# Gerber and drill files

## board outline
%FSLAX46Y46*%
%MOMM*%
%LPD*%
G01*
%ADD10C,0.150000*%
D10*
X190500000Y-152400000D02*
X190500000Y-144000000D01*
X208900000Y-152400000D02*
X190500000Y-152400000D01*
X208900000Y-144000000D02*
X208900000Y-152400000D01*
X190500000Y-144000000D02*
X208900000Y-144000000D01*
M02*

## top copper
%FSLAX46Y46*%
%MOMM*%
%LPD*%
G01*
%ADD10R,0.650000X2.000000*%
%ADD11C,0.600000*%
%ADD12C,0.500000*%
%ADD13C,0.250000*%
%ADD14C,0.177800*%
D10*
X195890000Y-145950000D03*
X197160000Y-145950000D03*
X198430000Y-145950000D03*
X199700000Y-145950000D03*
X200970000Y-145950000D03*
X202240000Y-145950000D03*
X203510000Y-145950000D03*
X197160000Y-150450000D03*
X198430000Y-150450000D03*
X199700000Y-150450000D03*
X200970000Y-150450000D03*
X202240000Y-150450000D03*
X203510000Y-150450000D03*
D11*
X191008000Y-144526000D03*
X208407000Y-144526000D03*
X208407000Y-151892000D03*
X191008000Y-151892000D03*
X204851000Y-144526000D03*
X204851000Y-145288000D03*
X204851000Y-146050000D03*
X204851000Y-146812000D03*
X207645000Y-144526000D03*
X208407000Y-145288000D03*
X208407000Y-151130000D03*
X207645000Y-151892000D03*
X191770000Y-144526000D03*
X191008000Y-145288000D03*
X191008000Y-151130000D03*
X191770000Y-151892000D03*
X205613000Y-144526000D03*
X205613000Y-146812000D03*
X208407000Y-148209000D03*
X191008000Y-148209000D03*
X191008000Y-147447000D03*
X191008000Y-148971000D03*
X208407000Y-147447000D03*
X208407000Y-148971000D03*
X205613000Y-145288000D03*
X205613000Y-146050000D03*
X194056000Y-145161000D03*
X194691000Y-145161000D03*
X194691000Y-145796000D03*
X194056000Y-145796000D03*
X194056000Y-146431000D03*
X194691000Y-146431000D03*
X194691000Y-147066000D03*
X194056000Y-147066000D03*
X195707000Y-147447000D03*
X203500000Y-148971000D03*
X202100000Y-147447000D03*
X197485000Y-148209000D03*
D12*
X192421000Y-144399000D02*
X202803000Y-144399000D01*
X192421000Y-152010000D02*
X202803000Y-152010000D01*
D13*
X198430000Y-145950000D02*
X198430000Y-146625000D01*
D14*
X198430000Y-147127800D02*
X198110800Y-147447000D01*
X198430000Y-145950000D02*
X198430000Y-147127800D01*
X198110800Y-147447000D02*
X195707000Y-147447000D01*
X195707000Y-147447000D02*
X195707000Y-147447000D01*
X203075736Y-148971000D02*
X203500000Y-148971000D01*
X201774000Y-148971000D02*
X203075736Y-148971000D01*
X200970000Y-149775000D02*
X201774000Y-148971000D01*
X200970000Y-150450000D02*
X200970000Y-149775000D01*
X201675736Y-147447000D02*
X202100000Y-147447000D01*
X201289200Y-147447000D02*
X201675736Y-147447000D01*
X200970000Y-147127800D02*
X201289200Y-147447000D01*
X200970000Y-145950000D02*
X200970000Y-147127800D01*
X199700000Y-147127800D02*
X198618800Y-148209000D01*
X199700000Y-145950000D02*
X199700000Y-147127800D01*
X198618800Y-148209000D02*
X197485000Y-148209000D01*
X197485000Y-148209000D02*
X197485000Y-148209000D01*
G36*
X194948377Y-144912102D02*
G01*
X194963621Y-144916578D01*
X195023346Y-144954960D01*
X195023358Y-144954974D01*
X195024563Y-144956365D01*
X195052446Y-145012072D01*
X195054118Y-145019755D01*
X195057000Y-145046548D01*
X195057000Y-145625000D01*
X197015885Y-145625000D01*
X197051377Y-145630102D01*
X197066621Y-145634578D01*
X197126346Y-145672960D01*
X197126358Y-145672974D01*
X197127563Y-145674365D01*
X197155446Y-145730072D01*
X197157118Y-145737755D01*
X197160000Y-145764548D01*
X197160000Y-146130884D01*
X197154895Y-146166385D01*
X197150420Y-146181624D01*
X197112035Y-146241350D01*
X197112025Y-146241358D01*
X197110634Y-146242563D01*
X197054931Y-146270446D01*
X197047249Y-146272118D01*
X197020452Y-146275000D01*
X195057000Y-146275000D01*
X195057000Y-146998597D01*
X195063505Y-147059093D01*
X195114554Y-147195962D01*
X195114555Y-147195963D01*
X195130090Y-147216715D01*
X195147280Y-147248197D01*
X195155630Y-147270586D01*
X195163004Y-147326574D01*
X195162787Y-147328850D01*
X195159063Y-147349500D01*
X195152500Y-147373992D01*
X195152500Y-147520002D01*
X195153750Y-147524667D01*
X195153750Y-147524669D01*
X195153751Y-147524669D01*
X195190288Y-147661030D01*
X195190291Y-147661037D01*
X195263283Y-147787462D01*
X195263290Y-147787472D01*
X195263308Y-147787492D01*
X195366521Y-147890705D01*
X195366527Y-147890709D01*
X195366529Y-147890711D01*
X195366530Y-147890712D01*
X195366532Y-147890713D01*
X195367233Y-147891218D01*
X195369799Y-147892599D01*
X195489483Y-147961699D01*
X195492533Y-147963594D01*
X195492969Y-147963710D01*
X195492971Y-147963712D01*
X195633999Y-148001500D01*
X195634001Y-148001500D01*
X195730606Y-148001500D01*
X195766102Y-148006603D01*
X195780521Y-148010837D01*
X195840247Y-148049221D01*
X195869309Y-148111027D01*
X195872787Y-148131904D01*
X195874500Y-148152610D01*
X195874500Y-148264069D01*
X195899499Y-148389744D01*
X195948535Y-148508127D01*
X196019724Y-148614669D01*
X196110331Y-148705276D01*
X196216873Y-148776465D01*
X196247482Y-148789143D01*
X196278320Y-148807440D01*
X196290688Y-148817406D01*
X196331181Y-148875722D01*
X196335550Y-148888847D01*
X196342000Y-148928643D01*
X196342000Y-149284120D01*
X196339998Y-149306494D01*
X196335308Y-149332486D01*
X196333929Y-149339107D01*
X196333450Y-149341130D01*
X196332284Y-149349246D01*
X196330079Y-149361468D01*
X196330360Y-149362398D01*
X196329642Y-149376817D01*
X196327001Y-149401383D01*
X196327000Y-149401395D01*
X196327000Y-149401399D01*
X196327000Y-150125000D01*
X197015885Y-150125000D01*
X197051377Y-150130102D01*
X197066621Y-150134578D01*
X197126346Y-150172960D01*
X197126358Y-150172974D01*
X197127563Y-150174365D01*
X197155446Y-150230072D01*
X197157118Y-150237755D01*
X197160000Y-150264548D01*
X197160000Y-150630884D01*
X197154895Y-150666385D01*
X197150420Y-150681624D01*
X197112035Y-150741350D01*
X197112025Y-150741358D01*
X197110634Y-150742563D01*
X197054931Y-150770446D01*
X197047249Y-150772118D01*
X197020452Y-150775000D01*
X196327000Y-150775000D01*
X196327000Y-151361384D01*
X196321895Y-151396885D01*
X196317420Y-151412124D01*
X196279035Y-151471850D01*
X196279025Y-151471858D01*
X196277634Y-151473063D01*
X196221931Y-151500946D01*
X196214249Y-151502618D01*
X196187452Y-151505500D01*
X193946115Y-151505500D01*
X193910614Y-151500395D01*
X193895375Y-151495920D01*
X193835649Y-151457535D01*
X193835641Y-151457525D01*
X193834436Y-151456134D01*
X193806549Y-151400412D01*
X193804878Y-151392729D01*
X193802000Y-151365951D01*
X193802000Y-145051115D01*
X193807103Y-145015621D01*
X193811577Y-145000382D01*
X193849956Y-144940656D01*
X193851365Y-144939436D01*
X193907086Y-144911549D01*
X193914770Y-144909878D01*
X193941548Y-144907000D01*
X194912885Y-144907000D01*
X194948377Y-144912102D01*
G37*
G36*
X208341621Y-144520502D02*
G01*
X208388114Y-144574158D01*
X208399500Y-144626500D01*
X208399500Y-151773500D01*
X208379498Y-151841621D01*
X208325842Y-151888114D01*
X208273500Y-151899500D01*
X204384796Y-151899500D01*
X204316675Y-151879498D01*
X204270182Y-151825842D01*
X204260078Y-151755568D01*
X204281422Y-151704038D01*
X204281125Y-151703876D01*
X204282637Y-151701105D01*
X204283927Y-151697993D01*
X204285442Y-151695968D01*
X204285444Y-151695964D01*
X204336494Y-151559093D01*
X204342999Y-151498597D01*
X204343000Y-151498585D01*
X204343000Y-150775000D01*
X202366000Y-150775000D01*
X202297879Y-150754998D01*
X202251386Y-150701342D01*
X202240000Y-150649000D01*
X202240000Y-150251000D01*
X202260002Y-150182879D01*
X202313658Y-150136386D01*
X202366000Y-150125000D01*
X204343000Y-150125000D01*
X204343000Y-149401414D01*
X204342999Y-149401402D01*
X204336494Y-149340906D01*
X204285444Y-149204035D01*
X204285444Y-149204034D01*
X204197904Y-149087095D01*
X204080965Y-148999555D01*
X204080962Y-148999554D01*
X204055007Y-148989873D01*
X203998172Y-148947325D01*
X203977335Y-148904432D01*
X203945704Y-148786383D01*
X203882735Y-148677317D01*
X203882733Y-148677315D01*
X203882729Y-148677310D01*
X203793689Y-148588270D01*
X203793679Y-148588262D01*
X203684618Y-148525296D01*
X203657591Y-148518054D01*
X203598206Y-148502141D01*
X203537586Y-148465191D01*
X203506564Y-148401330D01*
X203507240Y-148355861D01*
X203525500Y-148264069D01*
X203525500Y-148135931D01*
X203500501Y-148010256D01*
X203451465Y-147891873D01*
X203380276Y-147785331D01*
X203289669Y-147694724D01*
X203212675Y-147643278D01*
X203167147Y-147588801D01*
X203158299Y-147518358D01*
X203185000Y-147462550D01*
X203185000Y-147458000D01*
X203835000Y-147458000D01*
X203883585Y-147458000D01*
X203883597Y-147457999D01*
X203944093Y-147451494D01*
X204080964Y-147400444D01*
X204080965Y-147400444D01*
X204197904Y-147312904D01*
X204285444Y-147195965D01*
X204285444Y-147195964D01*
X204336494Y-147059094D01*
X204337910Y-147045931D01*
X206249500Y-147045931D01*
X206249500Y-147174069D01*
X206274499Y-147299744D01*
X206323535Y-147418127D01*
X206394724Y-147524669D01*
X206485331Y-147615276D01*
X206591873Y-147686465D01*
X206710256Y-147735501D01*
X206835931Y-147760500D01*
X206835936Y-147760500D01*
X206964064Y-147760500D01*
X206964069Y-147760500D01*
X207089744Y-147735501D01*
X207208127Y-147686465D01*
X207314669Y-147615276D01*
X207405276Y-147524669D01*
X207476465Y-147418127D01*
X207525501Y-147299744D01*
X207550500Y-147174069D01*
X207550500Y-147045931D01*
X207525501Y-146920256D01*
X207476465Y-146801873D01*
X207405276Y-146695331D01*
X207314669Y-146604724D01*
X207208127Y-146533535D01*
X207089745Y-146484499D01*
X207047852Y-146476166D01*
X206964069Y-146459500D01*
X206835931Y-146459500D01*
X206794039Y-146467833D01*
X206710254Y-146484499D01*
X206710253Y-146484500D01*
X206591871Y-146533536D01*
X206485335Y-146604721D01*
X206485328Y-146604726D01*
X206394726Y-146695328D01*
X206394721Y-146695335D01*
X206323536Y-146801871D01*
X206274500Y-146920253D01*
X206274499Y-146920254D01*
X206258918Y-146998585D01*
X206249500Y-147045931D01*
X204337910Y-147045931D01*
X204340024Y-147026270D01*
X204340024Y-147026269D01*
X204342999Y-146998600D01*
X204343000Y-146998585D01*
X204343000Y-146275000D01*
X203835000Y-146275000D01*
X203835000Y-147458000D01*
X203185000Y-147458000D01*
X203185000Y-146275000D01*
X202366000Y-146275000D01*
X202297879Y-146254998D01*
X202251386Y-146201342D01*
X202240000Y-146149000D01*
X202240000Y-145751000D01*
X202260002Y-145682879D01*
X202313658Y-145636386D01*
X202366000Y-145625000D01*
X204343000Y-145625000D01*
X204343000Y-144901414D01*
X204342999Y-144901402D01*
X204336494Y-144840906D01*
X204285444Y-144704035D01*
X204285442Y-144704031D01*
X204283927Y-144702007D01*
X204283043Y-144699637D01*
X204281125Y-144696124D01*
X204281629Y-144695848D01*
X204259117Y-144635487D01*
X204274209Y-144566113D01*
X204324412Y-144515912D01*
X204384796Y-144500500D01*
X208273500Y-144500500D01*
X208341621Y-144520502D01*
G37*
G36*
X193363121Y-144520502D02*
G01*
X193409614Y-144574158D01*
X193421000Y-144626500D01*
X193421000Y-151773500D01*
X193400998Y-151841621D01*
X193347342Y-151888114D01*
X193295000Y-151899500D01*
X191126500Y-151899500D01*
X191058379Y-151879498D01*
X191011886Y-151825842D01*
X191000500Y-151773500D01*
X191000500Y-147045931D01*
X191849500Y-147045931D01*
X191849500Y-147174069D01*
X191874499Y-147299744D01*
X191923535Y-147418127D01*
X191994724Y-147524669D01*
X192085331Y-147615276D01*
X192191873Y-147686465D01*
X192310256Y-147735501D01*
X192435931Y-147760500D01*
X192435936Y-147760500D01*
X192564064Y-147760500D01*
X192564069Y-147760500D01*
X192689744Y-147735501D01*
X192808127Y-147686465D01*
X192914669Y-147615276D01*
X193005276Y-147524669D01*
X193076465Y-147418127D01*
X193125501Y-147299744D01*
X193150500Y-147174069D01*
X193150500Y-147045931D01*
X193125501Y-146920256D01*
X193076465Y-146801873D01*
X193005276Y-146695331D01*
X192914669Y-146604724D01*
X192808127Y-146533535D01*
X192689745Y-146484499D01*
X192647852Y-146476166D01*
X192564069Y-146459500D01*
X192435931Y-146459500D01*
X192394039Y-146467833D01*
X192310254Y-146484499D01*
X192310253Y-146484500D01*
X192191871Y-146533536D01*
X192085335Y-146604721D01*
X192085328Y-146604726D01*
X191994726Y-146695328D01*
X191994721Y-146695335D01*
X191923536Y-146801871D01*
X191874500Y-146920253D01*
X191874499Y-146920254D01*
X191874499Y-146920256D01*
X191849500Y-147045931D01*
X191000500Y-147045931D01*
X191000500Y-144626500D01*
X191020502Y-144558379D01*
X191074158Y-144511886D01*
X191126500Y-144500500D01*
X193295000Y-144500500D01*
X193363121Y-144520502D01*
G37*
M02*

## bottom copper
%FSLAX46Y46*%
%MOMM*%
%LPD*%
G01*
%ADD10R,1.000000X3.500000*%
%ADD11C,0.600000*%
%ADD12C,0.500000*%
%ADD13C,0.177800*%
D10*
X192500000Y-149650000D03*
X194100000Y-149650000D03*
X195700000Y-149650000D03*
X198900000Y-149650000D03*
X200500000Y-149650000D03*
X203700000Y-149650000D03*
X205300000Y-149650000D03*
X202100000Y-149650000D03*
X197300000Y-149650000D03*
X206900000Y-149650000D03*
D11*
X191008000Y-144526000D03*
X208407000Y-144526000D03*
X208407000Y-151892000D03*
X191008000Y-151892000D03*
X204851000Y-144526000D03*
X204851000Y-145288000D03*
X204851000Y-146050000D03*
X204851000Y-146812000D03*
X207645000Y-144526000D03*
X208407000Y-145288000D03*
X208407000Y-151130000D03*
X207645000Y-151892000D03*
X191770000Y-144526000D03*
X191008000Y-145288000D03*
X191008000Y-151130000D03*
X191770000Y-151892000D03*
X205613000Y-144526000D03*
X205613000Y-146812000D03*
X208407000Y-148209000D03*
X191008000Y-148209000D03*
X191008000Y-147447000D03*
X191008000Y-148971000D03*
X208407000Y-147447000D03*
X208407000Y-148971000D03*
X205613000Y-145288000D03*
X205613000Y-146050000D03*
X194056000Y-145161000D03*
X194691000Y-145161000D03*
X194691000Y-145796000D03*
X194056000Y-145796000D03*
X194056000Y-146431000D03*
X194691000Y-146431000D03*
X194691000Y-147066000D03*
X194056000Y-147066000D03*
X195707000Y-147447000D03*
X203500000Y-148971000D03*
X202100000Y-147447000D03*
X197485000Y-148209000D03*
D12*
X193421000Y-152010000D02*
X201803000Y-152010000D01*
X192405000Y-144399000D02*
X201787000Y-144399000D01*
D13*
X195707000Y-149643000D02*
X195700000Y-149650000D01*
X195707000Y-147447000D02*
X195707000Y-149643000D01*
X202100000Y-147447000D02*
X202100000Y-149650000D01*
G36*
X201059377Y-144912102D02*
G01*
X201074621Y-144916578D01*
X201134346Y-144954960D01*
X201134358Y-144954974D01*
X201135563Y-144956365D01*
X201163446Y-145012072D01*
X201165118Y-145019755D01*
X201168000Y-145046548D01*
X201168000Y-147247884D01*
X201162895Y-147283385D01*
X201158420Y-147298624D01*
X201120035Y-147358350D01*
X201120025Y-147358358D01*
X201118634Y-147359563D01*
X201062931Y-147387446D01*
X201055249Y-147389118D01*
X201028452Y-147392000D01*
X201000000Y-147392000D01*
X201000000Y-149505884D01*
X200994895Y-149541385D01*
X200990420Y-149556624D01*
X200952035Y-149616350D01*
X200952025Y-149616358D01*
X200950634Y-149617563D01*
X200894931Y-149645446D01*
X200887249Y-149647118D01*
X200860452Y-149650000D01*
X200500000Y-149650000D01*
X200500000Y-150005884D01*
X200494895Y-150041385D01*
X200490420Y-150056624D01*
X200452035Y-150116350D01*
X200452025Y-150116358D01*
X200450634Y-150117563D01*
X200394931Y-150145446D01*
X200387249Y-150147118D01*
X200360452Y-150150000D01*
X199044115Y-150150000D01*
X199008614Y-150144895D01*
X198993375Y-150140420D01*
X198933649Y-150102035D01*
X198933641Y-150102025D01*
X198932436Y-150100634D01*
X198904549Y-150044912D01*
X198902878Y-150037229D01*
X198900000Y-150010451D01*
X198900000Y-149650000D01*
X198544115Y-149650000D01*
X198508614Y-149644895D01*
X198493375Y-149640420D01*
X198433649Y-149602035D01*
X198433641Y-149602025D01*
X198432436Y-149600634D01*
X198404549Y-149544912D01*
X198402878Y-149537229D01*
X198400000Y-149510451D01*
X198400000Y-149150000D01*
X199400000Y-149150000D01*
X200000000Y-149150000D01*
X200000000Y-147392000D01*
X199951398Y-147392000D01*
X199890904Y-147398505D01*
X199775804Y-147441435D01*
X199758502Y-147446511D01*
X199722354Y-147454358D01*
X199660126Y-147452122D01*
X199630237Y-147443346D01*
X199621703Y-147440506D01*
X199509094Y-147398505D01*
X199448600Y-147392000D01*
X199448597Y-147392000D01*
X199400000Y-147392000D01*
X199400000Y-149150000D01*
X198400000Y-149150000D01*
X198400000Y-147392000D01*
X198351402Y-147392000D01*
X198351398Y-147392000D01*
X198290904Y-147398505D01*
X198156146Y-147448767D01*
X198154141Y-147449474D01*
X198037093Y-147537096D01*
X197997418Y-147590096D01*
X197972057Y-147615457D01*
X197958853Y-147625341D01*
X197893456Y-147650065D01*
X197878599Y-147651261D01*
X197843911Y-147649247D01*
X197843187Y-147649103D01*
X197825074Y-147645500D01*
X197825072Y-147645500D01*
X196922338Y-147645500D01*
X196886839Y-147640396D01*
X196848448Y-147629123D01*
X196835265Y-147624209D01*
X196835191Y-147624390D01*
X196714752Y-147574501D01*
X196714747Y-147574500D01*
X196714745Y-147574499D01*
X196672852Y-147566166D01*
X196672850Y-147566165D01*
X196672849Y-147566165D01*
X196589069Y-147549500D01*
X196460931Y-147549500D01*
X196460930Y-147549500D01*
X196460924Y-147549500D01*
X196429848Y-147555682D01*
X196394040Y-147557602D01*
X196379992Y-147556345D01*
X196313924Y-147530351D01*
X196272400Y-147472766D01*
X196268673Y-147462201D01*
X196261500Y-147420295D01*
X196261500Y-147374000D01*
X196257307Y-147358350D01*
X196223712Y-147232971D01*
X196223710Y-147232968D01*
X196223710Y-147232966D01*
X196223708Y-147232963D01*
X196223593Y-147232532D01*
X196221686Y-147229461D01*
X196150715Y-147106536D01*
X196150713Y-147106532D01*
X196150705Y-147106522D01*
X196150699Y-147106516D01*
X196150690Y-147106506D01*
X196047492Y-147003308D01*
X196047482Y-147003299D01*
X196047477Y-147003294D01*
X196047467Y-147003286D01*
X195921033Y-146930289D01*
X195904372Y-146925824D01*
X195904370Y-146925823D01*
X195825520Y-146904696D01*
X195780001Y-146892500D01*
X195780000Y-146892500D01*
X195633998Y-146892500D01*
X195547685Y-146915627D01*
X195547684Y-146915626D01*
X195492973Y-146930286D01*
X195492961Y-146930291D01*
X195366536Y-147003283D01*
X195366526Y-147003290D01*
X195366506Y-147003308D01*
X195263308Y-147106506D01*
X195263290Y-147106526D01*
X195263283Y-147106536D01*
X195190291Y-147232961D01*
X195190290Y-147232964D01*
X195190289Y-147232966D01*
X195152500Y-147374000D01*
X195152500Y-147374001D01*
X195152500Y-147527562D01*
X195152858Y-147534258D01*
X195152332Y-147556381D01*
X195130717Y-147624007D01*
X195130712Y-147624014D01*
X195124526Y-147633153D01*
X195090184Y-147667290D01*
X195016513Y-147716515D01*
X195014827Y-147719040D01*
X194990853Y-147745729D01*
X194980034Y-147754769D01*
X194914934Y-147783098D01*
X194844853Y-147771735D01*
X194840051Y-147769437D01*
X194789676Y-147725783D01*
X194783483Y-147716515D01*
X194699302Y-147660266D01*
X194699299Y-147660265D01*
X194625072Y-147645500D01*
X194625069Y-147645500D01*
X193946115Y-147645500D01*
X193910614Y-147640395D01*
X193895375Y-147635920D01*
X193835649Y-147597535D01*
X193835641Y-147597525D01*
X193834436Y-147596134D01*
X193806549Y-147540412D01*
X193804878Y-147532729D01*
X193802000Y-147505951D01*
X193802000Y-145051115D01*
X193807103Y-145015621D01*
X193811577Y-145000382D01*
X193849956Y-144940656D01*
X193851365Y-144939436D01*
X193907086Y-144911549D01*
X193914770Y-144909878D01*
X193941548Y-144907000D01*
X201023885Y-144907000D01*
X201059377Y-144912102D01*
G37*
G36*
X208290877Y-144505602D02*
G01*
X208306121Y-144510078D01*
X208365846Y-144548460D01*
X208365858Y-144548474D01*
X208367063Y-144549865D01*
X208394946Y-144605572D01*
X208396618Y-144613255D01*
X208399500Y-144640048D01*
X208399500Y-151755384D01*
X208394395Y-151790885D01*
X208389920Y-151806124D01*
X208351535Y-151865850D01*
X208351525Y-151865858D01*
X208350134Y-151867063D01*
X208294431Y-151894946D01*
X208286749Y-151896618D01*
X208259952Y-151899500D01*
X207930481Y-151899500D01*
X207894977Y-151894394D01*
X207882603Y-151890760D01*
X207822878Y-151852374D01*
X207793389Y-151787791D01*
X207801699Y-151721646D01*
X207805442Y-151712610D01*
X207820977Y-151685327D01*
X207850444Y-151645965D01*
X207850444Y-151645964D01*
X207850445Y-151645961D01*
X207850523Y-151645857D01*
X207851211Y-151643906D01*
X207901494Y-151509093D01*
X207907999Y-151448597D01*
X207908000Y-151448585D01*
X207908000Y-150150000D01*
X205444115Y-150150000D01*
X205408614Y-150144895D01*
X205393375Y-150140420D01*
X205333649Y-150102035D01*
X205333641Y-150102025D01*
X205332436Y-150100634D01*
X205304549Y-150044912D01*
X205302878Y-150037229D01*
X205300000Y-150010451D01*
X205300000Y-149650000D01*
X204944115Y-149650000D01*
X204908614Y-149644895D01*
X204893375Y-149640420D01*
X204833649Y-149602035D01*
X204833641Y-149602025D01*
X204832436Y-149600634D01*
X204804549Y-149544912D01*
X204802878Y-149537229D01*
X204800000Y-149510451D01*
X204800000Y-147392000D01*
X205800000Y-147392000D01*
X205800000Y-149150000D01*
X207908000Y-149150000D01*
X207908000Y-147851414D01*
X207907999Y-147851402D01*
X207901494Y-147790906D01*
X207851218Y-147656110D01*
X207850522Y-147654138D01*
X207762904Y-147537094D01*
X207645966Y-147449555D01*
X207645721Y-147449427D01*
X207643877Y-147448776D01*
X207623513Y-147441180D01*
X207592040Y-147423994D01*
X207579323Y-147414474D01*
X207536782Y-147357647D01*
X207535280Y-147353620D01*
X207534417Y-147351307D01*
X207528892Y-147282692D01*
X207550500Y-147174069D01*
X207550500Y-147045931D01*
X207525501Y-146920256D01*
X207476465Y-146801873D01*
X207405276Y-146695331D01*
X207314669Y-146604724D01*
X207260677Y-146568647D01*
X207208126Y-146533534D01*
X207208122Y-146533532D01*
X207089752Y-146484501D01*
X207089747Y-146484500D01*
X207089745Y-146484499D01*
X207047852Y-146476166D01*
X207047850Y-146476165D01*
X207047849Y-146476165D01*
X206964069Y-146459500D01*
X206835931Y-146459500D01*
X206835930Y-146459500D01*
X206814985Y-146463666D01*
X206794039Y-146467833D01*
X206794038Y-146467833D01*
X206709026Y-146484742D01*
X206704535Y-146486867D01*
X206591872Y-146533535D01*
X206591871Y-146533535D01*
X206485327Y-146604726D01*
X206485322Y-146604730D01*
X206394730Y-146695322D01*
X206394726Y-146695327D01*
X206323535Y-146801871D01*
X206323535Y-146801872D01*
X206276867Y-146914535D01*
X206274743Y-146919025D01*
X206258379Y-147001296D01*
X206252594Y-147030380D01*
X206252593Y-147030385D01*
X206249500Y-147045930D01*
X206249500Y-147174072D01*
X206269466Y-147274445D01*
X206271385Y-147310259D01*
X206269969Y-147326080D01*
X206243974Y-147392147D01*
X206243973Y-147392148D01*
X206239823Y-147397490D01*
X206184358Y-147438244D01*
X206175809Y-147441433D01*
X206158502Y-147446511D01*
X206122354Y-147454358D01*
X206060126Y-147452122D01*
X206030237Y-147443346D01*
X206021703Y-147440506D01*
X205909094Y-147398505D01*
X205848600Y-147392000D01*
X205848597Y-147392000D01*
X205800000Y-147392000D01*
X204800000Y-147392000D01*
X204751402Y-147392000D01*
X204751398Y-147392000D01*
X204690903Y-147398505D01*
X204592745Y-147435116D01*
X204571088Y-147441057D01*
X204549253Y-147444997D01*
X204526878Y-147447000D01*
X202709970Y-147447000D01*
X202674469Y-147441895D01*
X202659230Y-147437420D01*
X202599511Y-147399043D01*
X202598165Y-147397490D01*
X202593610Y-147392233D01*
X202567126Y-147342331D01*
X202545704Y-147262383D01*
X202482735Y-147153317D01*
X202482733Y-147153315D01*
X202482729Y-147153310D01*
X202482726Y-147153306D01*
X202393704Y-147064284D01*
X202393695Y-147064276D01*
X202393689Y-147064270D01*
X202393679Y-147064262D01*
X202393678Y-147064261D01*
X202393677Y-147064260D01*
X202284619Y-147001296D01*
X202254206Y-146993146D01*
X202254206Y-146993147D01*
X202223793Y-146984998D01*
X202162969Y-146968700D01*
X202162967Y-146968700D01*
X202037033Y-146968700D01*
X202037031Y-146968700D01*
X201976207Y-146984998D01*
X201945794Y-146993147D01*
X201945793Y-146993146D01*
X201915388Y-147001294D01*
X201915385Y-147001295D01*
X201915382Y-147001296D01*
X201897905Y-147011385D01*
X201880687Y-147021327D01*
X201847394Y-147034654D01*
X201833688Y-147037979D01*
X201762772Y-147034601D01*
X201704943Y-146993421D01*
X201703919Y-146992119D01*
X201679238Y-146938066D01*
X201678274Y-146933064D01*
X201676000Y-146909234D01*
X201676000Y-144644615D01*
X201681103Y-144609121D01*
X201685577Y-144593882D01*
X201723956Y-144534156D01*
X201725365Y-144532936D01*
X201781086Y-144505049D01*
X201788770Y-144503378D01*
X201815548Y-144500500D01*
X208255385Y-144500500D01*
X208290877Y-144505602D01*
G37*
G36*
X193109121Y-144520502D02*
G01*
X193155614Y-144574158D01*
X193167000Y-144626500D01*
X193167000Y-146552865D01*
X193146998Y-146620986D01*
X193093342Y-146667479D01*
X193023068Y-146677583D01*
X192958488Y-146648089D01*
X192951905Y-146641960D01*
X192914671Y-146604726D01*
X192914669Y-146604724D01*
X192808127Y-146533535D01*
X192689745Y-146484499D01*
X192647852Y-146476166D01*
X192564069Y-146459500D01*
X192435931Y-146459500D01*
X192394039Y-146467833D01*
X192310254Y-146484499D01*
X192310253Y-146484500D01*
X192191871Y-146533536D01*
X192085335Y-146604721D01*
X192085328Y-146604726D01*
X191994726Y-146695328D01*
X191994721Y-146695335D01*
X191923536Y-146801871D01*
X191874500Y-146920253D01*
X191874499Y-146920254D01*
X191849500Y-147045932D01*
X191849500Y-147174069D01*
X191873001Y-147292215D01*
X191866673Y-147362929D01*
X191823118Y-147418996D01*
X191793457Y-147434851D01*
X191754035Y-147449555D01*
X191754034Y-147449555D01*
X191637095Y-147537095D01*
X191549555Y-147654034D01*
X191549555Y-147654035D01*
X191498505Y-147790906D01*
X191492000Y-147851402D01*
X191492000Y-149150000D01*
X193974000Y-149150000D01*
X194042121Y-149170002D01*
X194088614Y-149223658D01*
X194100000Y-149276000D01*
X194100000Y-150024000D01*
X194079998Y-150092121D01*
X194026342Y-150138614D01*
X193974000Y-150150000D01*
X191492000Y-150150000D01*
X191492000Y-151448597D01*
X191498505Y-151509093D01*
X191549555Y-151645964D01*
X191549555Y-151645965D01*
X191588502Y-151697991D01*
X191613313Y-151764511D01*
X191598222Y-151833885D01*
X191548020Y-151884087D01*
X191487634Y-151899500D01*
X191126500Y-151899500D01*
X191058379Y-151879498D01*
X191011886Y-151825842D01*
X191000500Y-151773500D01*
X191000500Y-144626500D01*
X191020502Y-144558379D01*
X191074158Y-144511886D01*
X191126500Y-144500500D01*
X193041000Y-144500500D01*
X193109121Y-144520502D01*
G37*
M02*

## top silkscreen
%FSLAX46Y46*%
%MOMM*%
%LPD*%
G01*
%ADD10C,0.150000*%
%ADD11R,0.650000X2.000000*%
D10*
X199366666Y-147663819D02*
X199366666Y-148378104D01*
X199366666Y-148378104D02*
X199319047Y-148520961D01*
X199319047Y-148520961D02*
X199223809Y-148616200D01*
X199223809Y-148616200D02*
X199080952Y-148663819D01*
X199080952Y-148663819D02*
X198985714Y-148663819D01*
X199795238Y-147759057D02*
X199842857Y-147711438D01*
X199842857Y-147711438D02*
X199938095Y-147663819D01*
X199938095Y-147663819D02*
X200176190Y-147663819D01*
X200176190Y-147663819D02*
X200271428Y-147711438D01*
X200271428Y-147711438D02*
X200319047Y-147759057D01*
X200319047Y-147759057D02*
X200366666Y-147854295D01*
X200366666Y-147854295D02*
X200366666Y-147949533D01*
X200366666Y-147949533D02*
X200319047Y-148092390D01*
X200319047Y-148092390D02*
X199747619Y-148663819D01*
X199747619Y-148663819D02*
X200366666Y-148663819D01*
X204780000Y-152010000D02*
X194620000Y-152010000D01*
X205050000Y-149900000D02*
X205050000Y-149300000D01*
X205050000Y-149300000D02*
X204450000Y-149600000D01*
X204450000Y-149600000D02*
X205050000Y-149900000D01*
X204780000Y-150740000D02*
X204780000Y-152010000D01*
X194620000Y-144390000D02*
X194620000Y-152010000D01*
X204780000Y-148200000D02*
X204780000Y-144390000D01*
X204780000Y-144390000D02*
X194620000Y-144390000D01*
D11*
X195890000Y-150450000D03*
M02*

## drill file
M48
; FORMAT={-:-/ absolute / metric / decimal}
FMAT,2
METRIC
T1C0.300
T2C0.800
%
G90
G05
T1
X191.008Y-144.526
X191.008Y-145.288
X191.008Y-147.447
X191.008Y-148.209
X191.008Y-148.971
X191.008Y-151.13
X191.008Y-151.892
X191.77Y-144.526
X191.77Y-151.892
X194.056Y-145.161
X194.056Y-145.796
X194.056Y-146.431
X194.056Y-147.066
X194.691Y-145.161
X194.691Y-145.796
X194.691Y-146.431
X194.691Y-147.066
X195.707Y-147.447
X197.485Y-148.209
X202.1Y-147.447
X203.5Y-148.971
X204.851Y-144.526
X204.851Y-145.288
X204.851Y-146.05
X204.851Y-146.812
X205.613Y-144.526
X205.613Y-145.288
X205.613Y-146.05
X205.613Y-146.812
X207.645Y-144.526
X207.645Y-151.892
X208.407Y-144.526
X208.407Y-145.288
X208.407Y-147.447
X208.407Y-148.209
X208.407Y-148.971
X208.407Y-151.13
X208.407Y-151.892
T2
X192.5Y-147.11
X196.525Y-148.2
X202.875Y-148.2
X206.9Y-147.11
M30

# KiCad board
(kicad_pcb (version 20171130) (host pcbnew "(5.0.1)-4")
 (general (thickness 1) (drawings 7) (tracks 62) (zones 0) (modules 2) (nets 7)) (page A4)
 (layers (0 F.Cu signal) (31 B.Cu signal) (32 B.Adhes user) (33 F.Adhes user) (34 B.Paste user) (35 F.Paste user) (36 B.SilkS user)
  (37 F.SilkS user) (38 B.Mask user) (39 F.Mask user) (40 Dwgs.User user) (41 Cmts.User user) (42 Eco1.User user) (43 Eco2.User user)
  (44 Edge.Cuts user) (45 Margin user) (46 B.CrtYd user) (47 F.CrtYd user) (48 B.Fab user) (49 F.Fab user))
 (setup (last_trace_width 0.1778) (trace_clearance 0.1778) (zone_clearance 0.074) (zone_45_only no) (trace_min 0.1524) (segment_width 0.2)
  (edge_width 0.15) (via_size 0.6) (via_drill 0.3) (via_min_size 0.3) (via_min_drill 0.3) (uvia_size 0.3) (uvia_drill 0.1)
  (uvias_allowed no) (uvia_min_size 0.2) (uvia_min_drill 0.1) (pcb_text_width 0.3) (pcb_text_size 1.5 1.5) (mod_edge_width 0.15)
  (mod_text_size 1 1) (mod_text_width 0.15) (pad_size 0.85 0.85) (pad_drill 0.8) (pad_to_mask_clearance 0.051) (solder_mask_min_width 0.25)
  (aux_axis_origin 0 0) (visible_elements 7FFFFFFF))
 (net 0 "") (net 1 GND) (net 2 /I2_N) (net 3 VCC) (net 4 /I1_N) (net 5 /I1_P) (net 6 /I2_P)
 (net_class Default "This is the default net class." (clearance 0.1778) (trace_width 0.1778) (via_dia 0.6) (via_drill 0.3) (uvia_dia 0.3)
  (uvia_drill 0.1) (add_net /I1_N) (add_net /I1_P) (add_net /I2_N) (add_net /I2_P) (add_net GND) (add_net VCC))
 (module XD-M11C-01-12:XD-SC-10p (layer B.Cu) (at 199.7 149.65 180)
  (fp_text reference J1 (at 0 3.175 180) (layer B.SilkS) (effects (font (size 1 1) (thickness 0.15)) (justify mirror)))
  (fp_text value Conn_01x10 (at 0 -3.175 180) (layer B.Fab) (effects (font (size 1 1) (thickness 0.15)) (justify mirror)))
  (pad 10 smd rect (at 7.2 0 180) (size 1 3.5) (layers B.Cu B.Paste B.Mask) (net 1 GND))
  (pad 9 smd rect (at 5.6 0 180) (size 1 3.5) (layers B.Cu B.Paste B.Mask) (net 1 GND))
  (pad 8 smd rect (at 4 0 180) (size 1 3.5) (layers B.Cu B.Paste B.Mask) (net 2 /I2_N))
  (pad 6 smd rect (at 0.8 0 180) (size 1 3.5) (layers B.Cu B.Paste B.Mask) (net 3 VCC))
  (pad 5 smd rect (at -0.8 0 180) (size 1 3.5) (layers B.Cu B.Paste B.Mask) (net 3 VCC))
  (pad 3 smd rect (at -4 0 180) (size 1 3.5) (layers B.Cu B.Paste B.Mask) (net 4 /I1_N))
  (pad 2 smd rect (at -5.6 0 180) (size 1 3.5) (layers B.Cu B.Paste B.Mask) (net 1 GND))
  (pad 4 smd rect (at -2.4 0 180) (size 1 3.5) (layers B.Cu B.Paste B.Mask) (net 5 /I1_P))
  (pad 7 smd rect (at 2.4 0 180) (size 1 3.5) (layers B.Cu B.Paste B.Mask) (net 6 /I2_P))
  (pad 1 smd rect (at -7.2 0 180) (size 1 3.5) (layers B.Cu B.Paste B.Mask) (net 1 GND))
  (pad "" np_thru_hole circle (at 7.2 2.54 180) (size 0.8 0.8) (drill 0.8) (layers *.Cu *.Mask) (clearance 0.1524))
  (pad "" np_thru_hole circle (at -7.2 2.54 180) (size 0.8 0.8) (drill 0.8) (layers *.Cu *.Mask) (clearance 0.1524)))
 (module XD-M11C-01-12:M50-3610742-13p (layer F.Cu) (at 199.7 148.2 180)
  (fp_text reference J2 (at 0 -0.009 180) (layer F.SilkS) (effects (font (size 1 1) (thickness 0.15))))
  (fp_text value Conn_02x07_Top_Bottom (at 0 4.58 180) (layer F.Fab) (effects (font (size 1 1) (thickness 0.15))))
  (fp_line (start -5.08 -3.81) (end 5.08 -3.81) (layer F.SilkS) (width 0.15))
  (fp_line (start -5.35 -1.7) (end -5.35 -1.1) (layer F.SilkS) (width 0.15))
  (fp_line (start -5.35 -1.1) (end -4.75 -1.4) (layer F.SilkS) (width 0.15))
  (fp_line (start -4.75 -1.4) (end -5.35 -1.7) (layer F.SilkS) (width 0.15))
  (fp_line (start -5.08 -2.54) (end -5.08 -3.81) (layer F.SilkS) (width 0.15))
  (fp_line (start 5.08 3.81) (end 5.08 -3.81) (layer F.SilkS) (width 0.15))
  (fp_line (start -5.08 0) (end -5.08 3.81) (layer F.SilkS) (width 0.15))
  (fp_line (start -5.08 3.81) (end 5.08 3.81) (layer F.SilkS) (width 0.15))
  (pad 14 smd rect (at 3.81 -2.25 180) (size 0.65 2) (layers F.SilkS))
  (pad "" np_thru_hole circle (at 3.175 0 180) (size 0.8 0.8) (drill 0.8) (layers *.Cu *.Mask) (clearance 0.1524))
  (pad "" np_thru_hole circle (at -3.175 0 180) (size 0.8 0.8) (drill 0.8) (layers *.Cu *.Mask) (clearance 0.1524))
  (pad 13 smd rect (at 3.81 2.25 180) (size 0.65 2) (layers F.Cu F.Paste F.Mask) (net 3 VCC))
  (pad 12 smd rect (at 2.54 2.25 180) (size 0.65 2) (layers F.Cu F.Paste F.Mask) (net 3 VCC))
  (pad 11 smd rect (at 1.27 2.25 180) (size 0.65 2) (layers F.Cu F.Paste F.Mask) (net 2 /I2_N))
  (pad 10 smd rect (at 0 2.25 180) (size 0.65 2) (layers F.Cu F.Paste F.Mask) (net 6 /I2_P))
  (pad 9 smd rect (at -1.27 2.25 180) (size 0.65 2) (layers F.Cu F.Paste F.Mask) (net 5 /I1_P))
  (pad 8 smd rect (at -2.54 2.25 180) (size 0.65 2) (layers F.Cu F.Paste F.Mask) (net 1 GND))
  (pad 7 smd rect (at -3.81 2.25 180) (size 0.65 2) (layers F.Cu F.Paste F.Mask) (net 1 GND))
  (pad 6 smd rect (at 2.54 -2.25 180) (size 0.65 2) (layers F.Cu F.Paste F.Mask) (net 3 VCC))
  (pad 5 smd rect (at 1.27 -2.25 180) (size 0.65 2) (layers F.Cu F.Paste F.Mask))
  (pad 4 smd rect (at 0 -2.25 180) (size 0.65 2) (layers F.Cu F.Paste F.Mask))
  (pad 3 smd rect (at -1.27 -2.25 180) (size 0.65 2) (layers F.Cu F.Paste F.Mask) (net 4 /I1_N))
  (pad 2 smd rect (at -2.54 -2.25 180) (size 0.65 2) (layers F.Cu F.Paste F.Mask) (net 1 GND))
  (pad 1 smd rect (at -3.81 -2.25 180) (size 0.65 2) (layers F.Cu F.Paste F.Mask) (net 1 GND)))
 (gr_line (start 190.5 152.4) (end 190.5 144) (layer Edge.Cuts) (width 0.15))
 (gr_line (start 208.9 152.4) (end 190.5 152.4) (layer Edge.Cuts) (width 0.15))
 (gr_line (start 208.9 144) (end 208.9 152.4) (layer Edge.Cuts) (width 0.15))
 (gr_line (start 190.5 144) (end 208.9 144) (layer Edge.Cuts) (width 0.15))
 (segment (start 192.421 144.399) (end 202.803 144.399) (width 0.5) (layer F.Cu) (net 1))
 (segment (start 193.421 152.01) (end 201.803 152.01) (width 0.5) (layer B.Cu) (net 1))
 (segment (start 192.405 144.399) (end 201.787 144.399) (width 0.5) (layer B.Cu) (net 1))
 (segment (start 192.421 152.01) (end 202.803 152.01) (width 0.5) (layer F.Cu) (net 1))
 (via (at 191.008 144.526) (size 0.6) (drill 0.3) (layers F.Cu B.Cu) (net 1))
 (via (at 208.407 144.526) (size 0.6) (drill 0.3) (layers F.Cu B.Cu) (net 1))
 (via (at 208.407 151.892) (size 0.6) (drill 0.3) (layers F.Cu B.Cu) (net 1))
 (via (at 191.008 151.892) (size 0.6) (drill 0.3) (layers F.Cu B.Cu) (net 1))
 (via (at 204.851 144.526) (size 0.6) (drill 0.3) (layers F.Cu B.Cu) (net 1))
 (via (at 204.851 145.288) (size 0.6) (drill 0.3) (layers F.Cu B.Cu) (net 1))
 (via (at 204.851 146.05) (size 0.6) (drill 0.3) (layers F.Cu B.Cu) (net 1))
 (via (at 204.851 146.812) (size 0.6) (drill 0.3) (layers F.Cu B.Cu) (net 1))
 (via (at 207.645 144.526) (size 0.6) (drill 0.3) (layers F.Cu B.Cu) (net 1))
 (via (at 208.407 145.288) (size 0.6) (drill 0.3) (layers F.Cu B.Cu) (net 1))
 (via (at 208.407 151.13) (size 0.6) (drill 0.3) (layers F.Cu B.Cu) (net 1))
 (via (at 207.645 151.892) (size 0.6) (drill 0.3) (layers F.Cu B.Cu) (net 1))
 (via (at 191.77 144.526) (size 0.6) (drill 0.3) (layers F.Cu B.Cu) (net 1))
 (via (at 191.008 145.288) (size 0.6) (drill 0.3) (layers F.Cu B.Cu) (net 1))
 (via (at 191.008 151.13) (size 0.6) (drill 0.3) (layers F.Cu B.Cu) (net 1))
 (via (at 191.77 151.892) (size 0.6) (drill 0.3) (layers F.Cu B.Cu) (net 1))
 (via (at 205.613 144.526) (size 0.6) (drill 0.3) (layers F.Cu B.Cu) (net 1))
 (via (at 205.613 146.812) (size 0.6) (drill 0.3) (layers F.Cu B.Cu) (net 1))
 (via (at 208.407 148.209) (size 0.6) (drill 0.3) (layers F.Cu B.Cu) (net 1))
 (via (at 191.008 148.209) (size 0.6) (drill 0.3) (layers F.Cu B.Cu) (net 1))
 (via (at 191.008 147.447) (size 0.6) (drill 0.3) (layers F.Cu B.Cu) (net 1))
 (via (at 191.008 148.971) (size 0.6) (drill 0.3) (layers F.Cu B.Cu) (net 1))
 (via (at 208.407 147.447) (size 0.6) (drill 0.3) (layers F.Cu B.Cu) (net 1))
 (via (at 208.407 148.971) (size 0.6) (drill 0.3) (layers F.Cu B.Cu) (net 1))
 (via (at 205.613 145.288) (size 0.6) (drill 0.3) (layers F.Cu B.Cu) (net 1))
 (via (at 205.613 146.05) (size 0.6) (drill 0.3) (layers F.Cu B.Cu) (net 1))
 (via (at 194.056 145.161) (size 0.6) (drill 0.3) (layers F.Cu B.Cu) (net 3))
 (via (at 194.691 145.161) (size 0.6) (drill 0.3) (layers F.Cu B.Cu) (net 3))
 (via (at 194.691 145.796) (size 0.6) (drill 0.3) (layers F.Cu B.Cu) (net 3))
 (via (at 194.056 145.796) (size 0.6) (drill 0.3) (layers F.Cu B.Cu) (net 3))
 (via (at 194.056 146.431) (size 0.6) (drill 0.3) (layers F.Cu B.Cu) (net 3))
 (via (at 194.691 146.431) (size 0.6) (drill 0.3) (layers F.Cu B.Cu) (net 3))
 (via (at 194.691 147.066) (size 0.6) (drill 0.3) (layers F.Cu B.Cu) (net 3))
 (via (at 194.056 147.066) (size 0.6) (drill 0.3) (layers F.Cu B.Cu) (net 3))
 (segment (start 198.43 145.95) (end 198.43 146.625) (width 0.25) (layer F.Cu) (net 2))
 (segment (start 198.43 147.1278) (end 198.1108 147.447) (width 0.1778) (layer F.Cu) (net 2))
 (segment (start 198.43 145.95) (end 198.43 147.1278) (width 0.1778) (layer F.Cu) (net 2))
 (segment (start 198.1108 147.447) (end 195.707 147.447) (width 0.1778) (layer F.Cu) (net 2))
 (segment (start 195.707 147.447) (end 195.707 147.447) (width 0.1778) (layer F.Cu) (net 2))
 (via (at 195.707 147.447) (size 0.6) (drill 0.3) (layers F.Cu B.Cu) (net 2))
 (segment (start 195.707 149.643) (end 195.7 149.65) (width 0.1778) (layer B.Cu) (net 2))
 (segment (start 195.707 147.447) (end 195.707 149.643) (width 0.1778) (layer B.Cu) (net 2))
 (via (at 203.5 148.971) (size 0.6) (drill 0.3) (layers F.Cu B.Cu) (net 4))
 (segment (start 203.075736 148.971) (end 203.5 148.971) (width 0.1778) (layer F.Cu) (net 4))
 (segment (start 201.774 148.971) (end 203.075736 148.971) (width 0.1778) (layer F.Cu) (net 4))
 (segment (start 200.97 149.775) (end 201.774 148.971) (width 0.1778) (layer F.Cu) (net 4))
 (segment (start 200.97 150.45) (end 200.97 149.775) (width 0.1778) (layer F.Cu) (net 4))
 (via (at 202.1 147.447) (size 0.6) (drill 0.3) (layers F.Cu B.Cu) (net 5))
 (segment (start 202.1 147.447) (end 202.1 149.65) (width 0.1778) (layer B.Cu) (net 5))
 (segment (start 201.675736 147.447) (end 202.1 147.447) (width 0.1778) (layer F.Cu) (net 5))
 (segment (start 201.2892 147.447) (end 201.675736 147.447) (width 0.1778) (layer F.Cu) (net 5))
 (segment (start 200.97 147.1278) (end 201.2892 147.447) (width 0.1778) (layer F.Cu) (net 5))
 (segment (start 200.97 145.95) (end 200.97 147.1278) (width 0.1778) (layer F.Cu) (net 5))
 (segment (start 199.7 147.1278) (end 198.6188 148.209) (width 0.1778) (layer F.Cu) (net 6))
 (segment (start 199.7 145.95) (end 199.7 147.1278) (width 0.1778) (layer F.Cu) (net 6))
 (segment (start 198.6188 148.209) (end 197.485 148.209) (width 0.1778) (layer F.Cu) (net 6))
 (segment (start 197.485 148.209) (end 197.485 148.209) (width 0.1778) (layer F.Cu) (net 6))
 (via (at 197.485 148.209) (size 0.6) (drill 0.3) (layers F.Cu B.Cu) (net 6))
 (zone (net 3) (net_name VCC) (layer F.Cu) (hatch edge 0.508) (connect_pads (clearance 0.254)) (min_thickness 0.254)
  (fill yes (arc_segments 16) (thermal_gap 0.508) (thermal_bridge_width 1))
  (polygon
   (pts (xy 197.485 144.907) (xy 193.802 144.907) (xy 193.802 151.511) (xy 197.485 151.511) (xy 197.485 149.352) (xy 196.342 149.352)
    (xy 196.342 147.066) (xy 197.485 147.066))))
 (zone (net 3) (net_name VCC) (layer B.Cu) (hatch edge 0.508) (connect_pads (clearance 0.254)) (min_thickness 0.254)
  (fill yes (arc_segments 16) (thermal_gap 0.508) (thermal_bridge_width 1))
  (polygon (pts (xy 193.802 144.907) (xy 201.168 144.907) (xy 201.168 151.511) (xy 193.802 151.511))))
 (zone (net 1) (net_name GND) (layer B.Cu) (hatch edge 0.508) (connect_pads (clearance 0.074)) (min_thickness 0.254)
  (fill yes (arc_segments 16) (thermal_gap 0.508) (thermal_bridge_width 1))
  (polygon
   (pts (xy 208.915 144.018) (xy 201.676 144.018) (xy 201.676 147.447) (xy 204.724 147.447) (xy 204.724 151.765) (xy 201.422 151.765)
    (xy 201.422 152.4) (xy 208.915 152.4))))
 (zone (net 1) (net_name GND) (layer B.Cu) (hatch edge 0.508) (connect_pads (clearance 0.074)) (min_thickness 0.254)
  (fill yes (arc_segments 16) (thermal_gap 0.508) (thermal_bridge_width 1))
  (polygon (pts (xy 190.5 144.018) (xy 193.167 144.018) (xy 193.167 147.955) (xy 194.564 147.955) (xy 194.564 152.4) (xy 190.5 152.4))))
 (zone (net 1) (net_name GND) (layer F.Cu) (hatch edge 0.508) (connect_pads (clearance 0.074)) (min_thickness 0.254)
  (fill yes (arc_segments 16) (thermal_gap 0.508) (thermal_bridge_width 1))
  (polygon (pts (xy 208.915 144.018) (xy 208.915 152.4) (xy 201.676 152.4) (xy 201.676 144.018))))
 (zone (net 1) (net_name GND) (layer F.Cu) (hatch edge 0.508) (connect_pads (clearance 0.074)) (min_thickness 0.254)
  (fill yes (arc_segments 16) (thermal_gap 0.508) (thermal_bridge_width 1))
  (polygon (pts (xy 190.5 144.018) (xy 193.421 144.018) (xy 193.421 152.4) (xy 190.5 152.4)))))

